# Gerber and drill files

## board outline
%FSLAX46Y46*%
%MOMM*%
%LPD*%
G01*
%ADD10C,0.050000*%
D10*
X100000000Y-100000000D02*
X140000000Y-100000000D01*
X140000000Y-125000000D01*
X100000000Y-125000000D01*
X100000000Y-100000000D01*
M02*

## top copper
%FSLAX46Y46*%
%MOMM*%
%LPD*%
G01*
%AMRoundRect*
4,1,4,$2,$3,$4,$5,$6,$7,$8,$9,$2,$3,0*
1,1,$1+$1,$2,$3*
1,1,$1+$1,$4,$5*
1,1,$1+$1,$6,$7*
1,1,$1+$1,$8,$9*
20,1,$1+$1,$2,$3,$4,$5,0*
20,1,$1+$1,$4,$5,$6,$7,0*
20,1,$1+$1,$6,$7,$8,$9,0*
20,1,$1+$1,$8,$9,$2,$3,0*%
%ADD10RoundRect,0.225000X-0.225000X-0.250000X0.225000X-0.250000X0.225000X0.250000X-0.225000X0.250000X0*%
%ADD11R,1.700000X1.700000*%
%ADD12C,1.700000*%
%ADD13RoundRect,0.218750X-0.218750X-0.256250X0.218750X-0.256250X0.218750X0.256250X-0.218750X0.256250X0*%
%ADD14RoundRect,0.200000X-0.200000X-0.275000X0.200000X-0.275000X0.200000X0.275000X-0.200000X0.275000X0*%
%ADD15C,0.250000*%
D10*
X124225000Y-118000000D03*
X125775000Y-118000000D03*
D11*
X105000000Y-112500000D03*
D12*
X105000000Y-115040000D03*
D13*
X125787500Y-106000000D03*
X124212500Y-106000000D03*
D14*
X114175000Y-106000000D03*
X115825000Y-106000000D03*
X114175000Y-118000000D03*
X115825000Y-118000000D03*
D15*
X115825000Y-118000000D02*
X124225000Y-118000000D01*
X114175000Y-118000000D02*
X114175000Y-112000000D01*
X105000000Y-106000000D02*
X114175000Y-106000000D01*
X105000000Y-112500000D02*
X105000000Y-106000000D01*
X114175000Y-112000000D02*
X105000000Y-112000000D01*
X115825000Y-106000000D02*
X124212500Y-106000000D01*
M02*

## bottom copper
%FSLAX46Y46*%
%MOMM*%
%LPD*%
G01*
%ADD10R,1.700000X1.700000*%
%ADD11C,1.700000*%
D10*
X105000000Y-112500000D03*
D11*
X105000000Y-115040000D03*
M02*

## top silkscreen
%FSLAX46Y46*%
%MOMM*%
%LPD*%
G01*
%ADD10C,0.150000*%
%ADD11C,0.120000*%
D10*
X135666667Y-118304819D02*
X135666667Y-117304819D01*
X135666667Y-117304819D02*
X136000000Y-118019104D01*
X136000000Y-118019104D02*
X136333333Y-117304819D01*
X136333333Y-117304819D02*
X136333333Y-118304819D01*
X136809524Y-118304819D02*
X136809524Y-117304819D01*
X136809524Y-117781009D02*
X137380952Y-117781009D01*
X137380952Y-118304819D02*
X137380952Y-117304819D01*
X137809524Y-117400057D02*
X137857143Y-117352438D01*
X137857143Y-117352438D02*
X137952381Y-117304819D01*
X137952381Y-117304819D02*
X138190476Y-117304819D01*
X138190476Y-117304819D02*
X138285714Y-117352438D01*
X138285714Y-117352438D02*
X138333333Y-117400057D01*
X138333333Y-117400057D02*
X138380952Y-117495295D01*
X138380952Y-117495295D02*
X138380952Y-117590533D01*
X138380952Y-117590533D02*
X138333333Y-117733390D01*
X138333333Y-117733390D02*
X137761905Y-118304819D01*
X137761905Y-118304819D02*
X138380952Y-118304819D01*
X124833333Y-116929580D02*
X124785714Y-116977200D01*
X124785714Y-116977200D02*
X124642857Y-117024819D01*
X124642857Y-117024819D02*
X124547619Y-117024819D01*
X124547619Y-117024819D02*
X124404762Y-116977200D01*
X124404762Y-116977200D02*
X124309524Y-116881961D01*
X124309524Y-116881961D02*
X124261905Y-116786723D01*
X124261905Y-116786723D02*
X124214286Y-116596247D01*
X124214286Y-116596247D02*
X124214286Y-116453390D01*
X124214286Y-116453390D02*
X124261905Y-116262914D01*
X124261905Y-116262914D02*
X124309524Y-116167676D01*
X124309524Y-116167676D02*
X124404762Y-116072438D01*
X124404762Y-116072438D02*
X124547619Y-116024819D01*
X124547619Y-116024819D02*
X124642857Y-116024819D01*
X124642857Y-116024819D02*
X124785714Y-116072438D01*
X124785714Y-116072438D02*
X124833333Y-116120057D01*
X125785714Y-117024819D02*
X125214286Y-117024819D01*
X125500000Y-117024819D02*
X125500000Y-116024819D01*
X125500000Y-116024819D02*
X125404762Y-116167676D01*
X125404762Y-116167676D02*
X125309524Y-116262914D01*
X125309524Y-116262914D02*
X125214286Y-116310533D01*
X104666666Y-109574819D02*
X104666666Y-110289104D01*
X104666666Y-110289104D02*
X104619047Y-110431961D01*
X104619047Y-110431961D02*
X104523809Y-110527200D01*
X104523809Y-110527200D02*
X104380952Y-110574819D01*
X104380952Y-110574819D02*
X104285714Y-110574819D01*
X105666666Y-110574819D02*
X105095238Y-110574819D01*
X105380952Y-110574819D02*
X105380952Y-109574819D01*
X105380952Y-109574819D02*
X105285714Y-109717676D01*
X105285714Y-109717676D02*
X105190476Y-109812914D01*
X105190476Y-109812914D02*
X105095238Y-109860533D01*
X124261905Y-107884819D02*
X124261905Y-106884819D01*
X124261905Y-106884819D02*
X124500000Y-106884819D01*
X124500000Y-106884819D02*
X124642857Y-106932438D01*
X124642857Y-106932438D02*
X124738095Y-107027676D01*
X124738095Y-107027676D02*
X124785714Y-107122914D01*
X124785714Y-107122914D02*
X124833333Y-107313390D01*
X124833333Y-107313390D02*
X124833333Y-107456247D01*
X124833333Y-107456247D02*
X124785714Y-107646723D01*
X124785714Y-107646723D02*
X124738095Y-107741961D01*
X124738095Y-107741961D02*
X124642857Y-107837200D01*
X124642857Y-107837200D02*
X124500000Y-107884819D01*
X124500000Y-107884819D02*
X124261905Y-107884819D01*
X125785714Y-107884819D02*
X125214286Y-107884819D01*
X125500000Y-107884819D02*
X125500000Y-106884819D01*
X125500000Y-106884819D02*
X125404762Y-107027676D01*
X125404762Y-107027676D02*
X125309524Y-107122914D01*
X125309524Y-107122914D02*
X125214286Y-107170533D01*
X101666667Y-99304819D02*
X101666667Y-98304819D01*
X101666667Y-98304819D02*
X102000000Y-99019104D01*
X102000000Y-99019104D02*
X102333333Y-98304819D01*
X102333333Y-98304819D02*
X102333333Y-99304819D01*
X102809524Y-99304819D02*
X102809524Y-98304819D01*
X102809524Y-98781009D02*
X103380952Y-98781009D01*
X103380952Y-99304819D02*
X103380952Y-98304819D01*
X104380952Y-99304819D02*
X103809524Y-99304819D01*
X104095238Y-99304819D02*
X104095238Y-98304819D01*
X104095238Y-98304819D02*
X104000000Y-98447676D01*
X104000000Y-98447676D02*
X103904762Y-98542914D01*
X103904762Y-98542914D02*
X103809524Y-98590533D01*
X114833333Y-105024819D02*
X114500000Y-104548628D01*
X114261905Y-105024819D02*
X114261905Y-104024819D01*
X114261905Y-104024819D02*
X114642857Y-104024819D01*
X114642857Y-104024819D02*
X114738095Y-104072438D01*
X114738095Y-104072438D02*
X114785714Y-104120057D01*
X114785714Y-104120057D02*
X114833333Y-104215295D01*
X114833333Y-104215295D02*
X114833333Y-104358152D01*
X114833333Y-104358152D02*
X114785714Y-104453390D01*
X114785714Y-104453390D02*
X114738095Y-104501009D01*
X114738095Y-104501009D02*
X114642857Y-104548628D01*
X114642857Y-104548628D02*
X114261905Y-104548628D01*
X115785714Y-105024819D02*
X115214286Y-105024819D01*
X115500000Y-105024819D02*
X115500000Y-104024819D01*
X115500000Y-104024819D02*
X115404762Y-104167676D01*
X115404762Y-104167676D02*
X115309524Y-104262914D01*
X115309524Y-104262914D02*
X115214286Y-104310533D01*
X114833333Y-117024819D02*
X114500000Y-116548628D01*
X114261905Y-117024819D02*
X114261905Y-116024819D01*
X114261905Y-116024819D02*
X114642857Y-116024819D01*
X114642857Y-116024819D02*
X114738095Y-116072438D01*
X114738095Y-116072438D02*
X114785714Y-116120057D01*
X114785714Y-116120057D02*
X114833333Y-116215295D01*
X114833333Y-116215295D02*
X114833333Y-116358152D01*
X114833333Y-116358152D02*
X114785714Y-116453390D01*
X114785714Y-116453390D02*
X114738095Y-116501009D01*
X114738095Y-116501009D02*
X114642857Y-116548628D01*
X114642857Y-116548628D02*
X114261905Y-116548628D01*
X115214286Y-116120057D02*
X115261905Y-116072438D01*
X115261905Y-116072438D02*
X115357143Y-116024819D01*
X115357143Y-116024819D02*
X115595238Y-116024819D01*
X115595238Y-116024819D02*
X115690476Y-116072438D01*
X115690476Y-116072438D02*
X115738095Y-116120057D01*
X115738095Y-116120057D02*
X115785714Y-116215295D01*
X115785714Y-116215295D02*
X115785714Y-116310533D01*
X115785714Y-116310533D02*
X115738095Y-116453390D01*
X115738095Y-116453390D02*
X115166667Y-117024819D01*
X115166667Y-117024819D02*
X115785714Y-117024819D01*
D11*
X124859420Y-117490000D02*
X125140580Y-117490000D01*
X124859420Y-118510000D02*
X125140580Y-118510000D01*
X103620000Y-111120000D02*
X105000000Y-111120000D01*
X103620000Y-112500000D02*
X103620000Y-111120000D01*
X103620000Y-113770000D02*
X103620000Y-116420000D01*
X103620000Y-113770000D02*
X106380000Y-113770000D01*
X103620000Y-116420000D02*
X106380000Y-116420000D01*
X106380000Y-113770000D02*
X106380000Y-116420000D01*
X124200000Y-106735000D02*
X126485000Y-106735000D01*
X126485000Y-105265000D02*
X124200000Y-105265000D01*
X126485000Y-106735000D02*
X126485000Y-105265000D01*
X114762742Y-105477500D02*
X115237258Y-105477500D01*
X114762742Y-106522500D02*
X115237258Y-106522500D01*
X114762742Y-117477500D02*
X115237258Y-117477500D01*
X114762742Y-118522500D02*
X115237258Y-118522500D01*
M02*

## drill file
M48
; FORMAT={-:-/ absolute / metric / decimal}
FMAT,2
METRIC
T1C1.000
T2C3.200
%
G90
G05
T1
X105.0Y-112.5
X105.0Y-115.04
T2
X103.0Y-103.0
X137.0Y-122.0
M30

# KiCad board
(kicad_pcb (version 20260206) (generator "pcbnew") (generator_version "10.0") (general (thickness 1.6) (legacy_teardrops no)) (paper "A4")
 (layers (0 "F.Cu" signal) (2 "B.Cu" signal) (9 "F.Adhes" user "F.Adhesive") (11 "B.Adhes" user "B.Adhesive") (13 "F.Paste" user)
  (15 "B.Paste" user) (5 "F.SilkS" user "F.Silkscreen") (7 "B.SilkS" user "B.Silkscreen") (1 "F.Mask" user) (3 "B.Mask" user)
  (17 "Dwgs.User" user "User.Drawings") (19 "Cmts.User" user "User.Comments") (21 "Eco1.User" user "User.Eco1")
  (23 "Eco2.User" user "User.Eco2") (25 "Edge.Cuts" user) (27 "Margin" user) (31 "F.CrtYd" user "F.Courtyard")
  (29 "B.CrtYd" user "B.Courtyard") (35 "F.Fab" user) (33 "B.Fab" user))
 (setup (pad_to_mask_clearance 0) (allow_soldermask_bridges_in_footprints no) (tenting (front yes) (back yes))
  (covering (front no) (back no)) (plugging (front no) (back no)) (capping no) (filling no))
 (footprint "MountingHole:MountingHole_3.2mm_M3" (layer "F.Cu") (at 137 122)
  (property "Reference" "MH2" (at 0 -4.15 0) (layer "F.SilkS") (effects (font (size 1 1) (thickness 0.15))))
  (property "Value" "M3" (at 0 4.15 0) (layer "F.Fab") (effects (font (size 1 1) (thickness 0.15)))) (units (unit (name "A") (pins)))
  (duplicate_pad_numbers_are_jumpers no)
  (pad "" np_thru_hole circle (at 0 0) (size 3.2 3.2) (drill 3.2) (layers "*.Cu" "*.Mask")))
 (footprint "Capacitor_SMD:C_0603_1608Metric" (layer "F.Cu") (at 125 118)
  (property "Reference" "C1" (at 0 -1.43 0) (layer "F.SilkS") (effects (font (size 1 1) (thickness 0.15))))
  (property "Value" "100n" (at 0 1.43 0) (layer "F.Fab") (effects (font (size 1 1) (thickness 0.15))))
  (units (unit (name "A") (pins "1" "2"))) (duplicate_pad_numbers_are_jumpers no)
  (fp_line (start -0.14058 -0.51) (end 0.14058 -0.51) (stroke (width 0.12) (type solid)) (layer "F.SilkS"))
  (fp_line (start -0.14058 0.51) (end 0.14058 0.51) (stroke (width 0.12) (type solid)) (layer "F.SilkS"))
  (pad "1" smd roundrect (at -0.775 0) (size 0.9 0.95) (layers "F.Cu" "F.Mask" "F.Paste") (roundrect_rratio 0.25) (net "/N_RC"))
  (pad "2" smd roundrect (at 0.775 0) (size 0.9 0.95) (layers "F.Cu" "F.Mask" "F.Paste") (roundrect_rratio 0.25) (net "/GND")))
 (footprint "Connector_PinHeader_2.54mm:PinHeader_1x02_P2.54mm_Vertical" (layer "F.Cu") (at 105 112.5)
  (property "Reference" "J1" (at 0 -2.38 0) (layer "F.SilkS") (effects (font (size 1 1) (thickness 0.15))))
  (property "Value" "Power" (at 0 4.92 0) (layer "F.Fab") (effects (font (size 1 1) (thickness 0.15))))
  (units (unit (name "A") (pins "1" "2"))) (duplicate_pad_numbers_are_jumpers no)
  (fp_line (start -1.38 -1.38) (end 0 -1.38) (stroke (width 0.12) (type solid)) (layer "F.SilkS"))
  (fp_line (start -1.38 0) (end -1.38 -1.38) (stroke (width 0.12) (type solid)) (layer "F.SilkS"))
  (fp_line (start -1.38 1.27) (end -1.38 3.92) (stroke (width 0.12) (type solid)) (layer "F.SilkS"))
  (fp_line (start -1.38 1.27) (end 1.38 1.27) (stroke (width 0.12) (type solid)) (layer "F.SilkS"))
  (fp_line (start -1.38 3.92) (end 1.38 3.92) (stroke (width 0.12) (type solid)) (layer "F.SilkS"))
  (fp_line (start 1.38 1.27) (end 1.38 3.92) (stroke (width 0.12) (type solid)) (layer "F.SilkS"))
  (pad "1" thru_hole rect (at 0 0) (size 1.7 1.7) (drill 1) (layers "*.Cu" "*.Mask") (remove_unused_layers no) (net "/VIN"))
  (pad "2" thru_hole circle (at 0 2.54) (size 1.7 1.7) (drill 1) (layers "*.Cu" "*.Mask") (remove_unused_layers no) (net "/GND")))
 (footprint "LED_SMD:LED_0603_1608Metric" (layer "F.Cu") (at 125 106 180)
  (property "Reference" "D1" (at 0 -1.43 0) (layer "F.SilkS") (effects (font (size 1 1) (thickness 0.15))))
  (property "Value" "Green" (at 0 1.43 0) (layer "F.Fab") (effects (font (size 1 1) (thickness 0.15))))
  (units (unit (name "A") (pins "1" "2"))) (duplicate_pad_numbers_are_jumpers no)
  (fp_line (start 0.8 -0.735) (end -1.485 -0.735) (stroke (width 0.12) (type solid)) (layer "F.SilkS"))
  (fp_line (start -1.485 0.735) (end 0.8 0.735) (stroke (width 0.12) (type solid)) (layer "F.SilkS"))
  (fp_line (start -1.485 -0.735) (end -1.485 0.735) (stroke (width 0.12) (type solid)) (layer "F.SilkS"))
  (pad "1" smd roundrect (at -0.7875 0) (size 0.875 0.95) (layers "F.Cu" "F.Mask" "F.Paste") (roundrect_rratio 0.25) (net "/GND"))
  (pad "2" smd roundrect (at 0.7875 0) (size 0.875 0.95) (layers "F.Cu" "F.Mask" "F.Paste") (roundrect_rratio 0.25) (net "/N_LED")))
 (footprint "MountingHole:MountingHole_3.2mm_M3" (layer "F.Cu") (at 103 103)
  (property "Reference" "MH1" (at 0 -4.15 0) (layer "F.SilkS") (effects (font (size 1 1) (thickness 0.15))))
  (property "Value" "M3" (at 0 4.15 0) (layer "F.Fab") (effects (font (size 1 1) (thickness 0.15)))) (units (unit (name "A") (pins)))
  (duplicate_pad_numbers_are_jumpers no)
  (pad "" np_thru_hole circle (at 0 0) (size 3.2 3.2) (drill 3.2) (layers "*.Cu" "*.Mask")))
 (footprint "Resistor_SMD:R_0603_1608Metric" (layer "F.Cu") (at 115 106)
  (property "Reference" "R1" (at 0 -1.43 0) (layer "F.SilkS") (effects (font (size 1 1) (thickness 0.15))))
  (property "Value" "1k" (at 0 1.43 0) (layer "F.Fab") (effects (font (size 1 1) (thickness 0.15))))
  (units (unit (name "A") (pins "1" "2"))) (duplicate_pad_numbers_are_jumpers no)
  (fp_line (start -0.237258 -0.5225) (end 0.237258 -0.5225) (stroke (width 0.12) (type solid)) (layer "F.SilkS"))
  (fp_line (start -0.237258 0.5225) (end 0.237258 0.5225) (stroke (width 0.12) (type solid)) (layer "F.SilkS"))
  (pad "1" smd roundrect (at -0.825 0) (size 0.8 0.95) (layers "F.Cu" "F.Mask" "F.Paste") (roundrect_rratio 0.25) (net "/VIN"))
  (pad "2" smd roundrect (at 0.825 0) (size 0.8 0.95) (layers "F.Cu" "F.Mask" "F.Paste") (roundrect_rratio 0.25) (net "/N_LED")))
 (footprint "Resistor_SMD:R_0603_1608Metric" (layer "F.Cu") (at 115 118)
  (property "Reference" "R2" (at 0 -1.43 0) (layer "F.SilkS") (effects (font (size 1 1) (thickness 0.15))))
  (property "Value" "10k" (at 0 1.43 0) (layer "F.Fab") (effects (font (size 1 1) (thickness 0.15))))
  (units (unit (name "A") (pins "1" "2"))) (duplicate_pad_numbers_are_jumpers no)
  (fp_line (start -0.237258 -0.5225) (end 0.237258 -0.5225) (stroke (width 0.12) (type solid)) (layer "F.SilkS"))
  (fp_line (start -0.237258 0.5225) (end 0.237258 0.5225) (stroke (width 0.12) (type solid)) (layer "F.SilkS"))
  (pad "1" smd roundrect (at -0.825 0) (size 0.8 0.95) (layers "F.Cu" "F.Mask" "F.Paste") (roundrect_rratio 0.25) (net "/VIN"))
  (pad "2" smd roundrect (at 0.825 0) (size 0.8 0.95) (layers "F.Cu" "F.Mask" "F.Paste") (roundrect_rratio 0.25) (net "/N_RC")))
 (gr_rect (start 100 100) (end 140 125) (stroke (width 0.05) (type default)) (fill no) (layer "Edge.Cuts"))
 (segment (start 115.825 118) (end 124.225 118) (width 0.25) (layer "F.Cu") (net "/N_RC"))
 (segment (start 114.175 118) (end 114.175 112) (width 0.25) (layer "F.Cu") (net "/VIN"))
 (segment (start 105 106) (end 114.175 106) (width 0.25) (layer "F.Cu") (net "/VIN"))
 (segment (start 105 112.5) (end 105 106) (width 0.25) (layer "F.Cu") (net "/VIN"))
 (segment (start 114.175 112) (end 105 112) (width 0.25) (layer "F.Cu") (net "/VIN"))
 (segment (start 115.825 106) (end 124.2125 106) (width 0.25) (layer "F.Cu") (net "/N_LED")))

